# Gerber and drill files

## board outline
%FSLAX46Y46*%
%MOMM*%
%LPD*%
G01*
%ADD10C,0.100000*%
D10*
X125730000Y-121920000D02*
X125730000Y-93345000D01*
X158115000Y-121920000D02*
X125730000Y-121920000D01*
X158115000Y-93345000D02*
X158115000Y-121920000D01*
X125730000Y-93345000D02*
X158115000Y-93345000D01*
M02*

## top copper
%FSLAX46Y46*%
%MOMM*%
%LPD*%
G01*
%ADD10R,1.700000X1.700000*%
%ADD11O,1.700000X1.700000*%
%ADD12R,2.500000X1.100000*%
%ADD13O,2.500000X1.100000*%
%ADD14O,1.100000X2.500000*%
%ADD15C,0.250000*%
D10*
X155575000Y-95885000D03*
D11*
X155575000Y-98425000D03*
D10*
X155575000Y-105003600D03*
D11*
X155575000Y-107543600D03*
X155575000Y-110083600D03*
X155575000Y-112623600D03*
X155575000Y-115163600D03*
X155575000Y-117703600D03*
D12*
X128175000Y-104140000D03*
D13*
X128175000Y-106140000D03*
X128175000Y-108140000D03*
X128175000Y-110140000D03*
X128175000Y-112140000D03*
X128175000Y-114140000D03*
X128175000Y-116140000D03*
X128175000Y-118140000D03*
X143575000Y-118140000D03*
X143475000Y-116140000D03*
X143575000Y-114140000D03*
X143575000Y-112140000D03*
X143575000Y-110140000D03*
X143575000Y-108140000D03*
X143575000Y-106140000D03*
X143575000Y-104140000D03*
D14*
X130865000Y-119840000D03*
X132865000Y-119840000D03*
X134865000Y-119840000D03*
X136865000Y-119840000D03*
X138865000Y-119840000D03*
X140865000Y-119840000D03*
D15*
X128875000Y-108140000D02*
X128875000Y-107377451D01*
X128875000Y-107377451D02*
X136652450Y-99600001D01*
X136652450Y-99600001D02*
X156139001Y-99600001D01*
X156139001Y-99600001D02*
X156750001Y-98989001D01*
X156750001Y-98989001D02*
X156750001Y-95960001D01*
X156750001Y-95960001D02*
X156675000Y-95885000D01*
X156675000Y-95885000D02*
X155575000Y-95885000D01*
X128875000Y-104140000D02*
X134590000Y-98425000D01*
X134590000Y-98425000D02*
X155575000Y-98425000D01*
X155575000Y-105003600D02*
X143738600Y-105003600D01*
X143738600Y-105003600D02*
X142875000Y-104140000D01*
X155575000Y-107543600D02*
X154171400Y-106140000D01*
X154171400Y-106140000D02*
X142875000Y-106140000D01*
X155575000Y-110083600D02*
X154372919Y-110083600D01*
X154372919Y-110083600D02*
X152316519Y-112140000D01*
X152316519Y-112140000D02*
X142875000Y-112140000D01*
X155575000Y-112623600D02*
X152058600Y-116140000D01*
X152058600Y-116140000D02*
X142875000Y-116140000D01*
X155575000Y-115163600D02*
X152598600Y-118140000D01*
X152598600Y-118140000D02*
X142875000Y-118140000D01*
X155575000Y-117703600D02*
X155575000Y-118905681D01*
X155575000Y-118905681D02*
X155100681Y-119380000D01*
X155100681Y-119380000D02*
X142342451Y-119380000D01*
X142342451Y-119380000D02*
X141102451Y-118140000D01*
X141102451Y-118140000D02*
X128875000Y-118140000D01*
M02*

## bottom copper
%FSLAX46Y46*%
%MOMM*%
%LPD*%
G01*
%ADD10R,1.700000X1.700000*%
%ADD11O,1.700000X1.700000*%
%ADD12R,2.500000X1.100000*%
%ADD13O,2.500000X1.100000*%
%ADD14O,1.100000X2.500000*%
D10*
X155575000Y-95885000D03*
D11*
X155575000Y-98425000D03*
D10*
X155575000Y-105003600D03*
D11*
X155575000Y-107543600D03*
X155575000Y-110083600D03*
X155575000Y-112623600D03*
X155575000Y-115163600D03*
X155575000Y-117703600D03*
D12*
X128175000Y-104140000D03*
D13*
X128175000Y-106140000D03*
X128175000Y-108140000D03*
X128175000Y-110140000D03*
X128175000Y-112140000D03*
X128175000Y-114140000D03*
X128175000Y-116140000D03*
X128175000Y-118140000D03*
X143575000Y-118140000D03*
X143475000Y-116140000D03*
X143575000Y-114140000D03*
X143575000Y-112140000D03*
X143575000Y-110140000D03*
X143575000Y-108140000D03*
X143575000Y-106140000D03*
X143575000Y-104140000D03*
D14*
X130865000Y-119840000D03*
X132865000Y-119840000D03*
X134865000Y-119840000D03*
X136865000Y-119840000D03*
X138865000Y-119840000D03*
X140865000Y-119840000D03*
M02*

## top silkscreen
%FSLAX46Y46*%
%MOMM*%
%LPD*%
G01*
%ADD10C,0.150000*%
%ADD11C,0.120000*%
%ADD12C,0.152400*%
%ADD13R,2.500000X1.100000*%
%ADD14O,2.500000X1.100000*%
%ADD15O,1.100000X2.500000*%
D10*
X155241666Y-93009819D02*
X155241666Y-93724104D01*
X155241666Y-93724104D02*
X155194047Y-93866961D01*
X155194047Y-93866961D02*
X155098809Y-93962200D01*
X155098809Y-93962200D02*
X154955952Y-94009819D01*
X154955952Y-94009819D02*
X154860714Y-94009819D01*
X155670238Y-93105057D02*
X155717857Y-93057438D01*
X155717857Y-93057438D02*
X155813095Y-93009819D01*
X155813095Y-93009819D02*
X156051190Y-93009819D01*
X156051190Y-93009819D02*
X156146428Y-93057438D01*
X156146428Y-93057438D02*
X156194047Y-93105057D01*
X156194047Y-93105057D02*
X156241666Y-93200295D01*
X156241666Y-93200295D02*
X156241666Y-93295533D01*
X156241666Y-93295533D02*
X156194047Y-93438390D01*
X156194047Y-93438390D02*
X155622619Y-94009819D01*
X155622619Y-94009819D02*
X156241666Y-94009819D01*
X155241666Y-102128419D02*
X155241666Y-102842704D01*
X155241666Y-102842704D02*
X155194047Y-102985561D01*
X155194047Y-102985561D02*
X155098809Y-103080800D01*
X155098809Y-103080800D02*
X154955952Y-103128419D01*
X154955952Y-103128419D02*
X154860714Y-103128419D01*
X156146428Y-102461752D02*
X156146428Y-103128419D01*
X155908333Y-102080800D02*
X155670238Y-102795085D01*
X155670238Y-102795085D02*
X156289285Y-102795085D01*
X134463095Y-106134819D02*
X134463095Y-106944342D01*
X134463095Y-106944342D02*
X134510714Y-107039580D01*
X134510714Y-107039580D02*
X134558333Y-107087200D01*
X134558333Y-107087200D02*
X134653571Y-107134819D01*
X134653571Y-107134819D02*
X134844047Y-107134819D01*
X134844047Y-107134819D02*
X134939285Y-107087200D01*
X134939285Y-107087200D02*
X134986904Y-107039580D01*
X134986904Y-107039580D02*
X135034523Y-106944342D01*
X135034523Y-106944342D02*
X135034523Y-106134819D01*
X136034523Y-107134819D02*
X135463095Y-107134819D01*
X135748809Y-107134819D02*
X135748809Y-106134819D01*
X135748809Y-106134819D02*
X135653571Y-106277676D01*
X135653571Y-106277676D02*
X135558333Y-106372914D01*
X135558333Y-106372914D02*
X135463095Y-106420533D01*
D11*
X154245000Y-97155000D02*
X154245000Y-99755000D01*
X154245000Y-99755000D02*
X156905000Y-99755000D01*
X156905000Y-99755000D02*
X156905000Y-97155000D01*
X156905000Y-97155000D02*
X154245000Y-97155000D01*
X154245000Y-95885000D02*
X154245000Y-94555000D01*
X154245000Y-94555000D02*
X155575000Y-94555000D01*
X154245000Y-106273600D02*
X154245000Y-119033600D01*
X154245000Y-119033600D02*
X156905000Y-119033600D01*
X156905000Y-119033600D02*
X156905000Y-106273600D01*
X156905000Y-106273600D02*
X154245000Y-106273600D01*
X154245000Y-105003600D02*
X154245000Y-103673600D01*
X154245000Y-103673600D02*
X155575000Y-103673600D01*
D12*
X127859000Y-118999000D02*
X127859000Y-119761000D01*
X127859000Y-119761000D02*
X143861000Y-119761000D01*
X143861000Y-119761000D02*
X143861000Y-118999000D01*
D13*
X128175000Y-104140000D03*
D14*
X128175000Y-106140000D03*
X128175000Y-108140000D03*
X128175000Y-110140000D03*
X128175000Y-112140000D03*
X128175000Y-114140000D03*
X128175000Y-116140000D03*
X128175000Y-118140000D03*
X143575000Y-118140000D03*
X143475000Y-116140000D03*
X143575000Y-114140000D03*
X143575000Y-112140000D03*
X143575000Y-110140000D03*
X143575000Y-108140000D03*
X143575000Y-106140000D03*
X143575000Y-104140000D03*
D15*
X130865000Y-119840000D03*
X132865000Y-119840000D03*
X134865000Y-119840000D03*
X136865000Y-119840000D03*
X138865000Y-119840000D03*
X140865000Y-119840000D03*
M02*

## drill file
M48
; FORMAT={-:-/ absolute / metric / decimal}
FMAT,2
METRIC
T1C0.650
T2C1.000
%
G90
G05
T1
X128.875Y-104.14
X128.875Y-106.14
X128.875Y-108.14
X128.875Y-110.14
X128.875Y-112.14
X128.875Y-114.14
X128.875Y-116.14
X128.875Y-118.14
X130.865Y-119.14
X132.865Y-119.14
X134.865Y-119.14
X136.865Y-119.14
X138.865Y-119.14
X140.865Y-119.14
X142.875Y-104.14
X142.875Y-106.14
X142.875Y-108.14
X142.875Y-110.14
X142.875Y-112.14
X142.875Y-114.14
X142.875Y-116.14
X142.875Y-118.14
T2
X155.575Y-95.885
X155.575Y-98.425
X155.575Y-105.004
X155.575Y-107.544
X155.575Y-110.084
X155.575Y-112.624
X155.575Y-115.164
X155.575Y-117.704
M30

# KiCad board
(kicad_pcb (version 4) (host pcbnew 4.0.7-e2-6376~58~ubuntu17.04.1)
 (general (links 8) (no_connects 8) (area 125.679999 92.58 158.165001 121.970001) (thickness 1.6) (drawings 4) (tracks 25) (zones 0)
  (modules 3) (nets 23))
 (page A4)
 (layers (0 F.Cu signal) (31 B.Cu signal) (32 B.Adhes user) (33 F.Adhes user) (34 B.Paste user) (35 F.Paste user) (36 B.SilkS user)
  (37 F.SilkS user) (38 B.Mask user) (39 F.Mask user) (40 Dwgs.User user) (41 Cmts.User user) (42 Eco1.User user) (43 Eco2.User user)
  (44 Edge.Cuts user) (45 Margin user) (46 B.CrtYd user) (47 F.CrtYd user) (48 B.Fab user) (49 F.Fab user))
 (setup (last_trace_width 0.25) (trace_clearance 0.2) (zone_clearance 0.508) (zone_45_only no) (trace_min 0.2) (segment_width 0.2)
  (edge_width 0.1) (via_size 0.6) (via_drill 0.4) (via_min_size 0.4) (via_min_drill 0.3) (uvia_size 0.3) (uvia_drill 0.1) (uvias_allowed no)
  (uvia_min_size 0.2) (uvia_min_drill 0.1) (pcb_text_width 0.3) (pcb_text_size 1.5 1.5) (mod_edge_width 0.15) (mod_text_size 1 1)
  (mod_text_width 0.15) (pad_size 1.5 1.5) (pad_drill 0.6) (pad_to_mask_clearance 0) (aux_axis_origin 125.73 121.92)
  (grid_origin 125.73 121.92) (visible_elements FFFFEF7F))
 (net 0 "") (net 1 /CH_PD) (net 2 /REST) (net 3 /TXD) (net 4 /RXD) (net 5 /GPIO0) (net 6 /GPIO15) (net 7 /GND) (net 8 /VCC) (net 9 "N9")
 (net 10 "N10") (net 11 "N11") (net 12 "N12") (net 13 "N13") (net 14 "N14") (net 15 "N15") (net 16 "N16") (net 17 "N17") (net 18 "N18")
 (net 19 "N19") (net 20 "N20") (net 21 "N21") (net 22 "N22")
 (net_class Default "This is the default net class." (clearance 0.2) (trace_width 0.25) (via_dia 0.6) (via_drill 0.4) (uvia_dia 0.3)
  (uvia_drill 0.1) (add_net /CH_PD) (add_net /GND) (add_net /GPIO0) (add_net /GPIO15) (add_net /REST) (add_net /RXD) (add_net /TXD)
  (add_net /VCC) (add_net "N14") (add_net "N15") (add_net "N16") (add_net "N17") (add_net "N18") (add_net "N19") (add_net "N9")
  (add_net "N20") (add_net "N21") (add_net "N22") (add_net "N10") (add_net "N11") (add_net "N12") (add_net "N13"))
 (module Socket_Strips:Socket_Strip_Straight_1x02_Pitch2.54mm (layer F.Cu) (at 155.575 95.885)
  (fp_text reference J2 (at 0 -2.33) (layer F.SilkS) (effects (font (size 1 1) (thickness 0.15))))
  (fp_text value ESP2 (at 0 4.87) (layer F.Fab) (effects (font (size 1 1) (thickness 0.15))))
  (fp_line (start -1.33 1.27) (end -1.33 3.87) (layer F.SilkS) (width 0.12))
  (fp_line (start -1.33 3.87) (end 1.33 3.87) (layer F.SilkS) (width 0.12))
  (fp_line (start 1.33 3.87) (end 1.33 1.27) (layer F.SilkS) (width 0.12))
  (fp_line (start 1.33 1.27) (end -1.33 1.27) (layer F.SilkS) (width 0.12))
  (fp_line (start -1.33 0) (end -1.33 -1.33) (layer F.SilkS) (width 0.12))
  (fp_line (start -1.33 -1.33) (end 0 -1.33) (layer F.SilkS) (width 0.12))
  (pad 1 thru_hole rect (at 0 0) (size 1.7 1.7) (drill 1) (layers *.Cu *.Mask) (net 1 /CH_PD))
  (pad 2 thru_hole oval (at 0 2.54) (size 1.7 1.7) (drill 1) (layers *.Cu *.Mask) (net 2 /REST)))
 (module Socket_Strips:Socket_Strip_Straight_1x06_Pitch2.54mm (layer F.Cu) (at 155.575 105.0036)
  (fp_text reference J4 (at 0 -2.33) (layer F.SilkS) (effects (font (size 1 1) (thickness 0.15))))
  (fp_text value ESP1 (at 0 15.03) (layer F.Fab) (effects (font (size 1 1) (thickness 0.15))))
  (fp_line (start -1.33 1.27) (end -1.33 14.03) (layer F.SilkS) (width 0.12))
  (fp_line (start -1.33 14.03) (end 1.33 14.03) (layer F.SilkS) (width 0.12))
  (fp_line (start 1.33 14.03) (end 1.33 1.27) (layer F.SilkS) (width 0.12))
  (fp_line (start 1.33 1.27) (end -1.33 1.27) (layer F.SilkS) (width 0.12))
  (fp_line (start -1.33 0) (end -1.33 -1.33) (layer F.SilkS) (width 0.12))
  (fp_line (start -1.33 -1.33) (end 0 -1.33) (layer F.SilkS) (width 0.12))
  (pad 1 thru_hole rect (at 0 0) (size 1.7 1.7) (drill 1) (layers *.Cu *.Mask) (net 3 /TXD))
  (pad 2 thru_hole oval (at 0 2.54) (size 1.7 1.7) (drill 1) (layers *.Cu *.Mask) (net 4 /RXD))
  (pad 3 thru_hole oval (at 0 5.08) (size 1.7 1.7) (drill 1) (layers *.Cu *.Mask) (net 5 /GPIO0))
  (pad 4 thru_hole oval (at 0 7.62) (size 1.7 1.7) (drill 1) (layers *.Cu *.Mask) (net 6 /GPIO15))
  (pad 5 thru_hole oval (at 0 10.16) (size 1.7 1.7) (drill 1) (layers *.Cu *.Mask) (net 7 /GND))
  (pad 6 thru_hole oval (at 0 12.7) (size 1.7 1.7) (drill 1) (layers *.Cu *.Mask) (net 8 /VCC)))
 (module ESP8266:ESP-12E (layer F.Cu) (at 128.875 104.14)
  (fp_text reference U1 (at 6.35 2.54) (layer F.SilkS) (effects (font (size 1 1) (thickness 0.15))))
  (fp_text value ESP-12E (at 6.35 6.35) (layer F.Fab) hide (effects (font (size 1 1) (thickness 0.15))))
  (fp_line (start -1.016 14.859) (end -1.016 15.621) (layer F.SilkS) (width 0.1524))
  (fp_line (start -1.016 15.621) (end 14.986 15.621) (layer F.SilkS) (width 0.1524))
  (fp_line (start 14.986 15.621) (end 14.986 14.859) (layer F.SilkS) (width 0.1524))
  (pad 1 thru_hole rect (at 0 0) (size 2.5 1.1) (drill 0.65 (offset -0.7 0)) (layers *.Cu *.Mask F.SilkS) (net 2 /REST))
  (pad 2 thru_hole oval (at 0 2) (size 2.5 1.1) (drill 0.65 (offset -0.7 0)) (layers *.Cu *.Mask F.SilkS) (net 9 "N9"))
  (pad 3 thru_hole oval (at 0 4) (size 2.5 1.1) (drill 0.65 (offset -0.7 0)) (layers *.Cu *.Mask F.SilkS) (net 1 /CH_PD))
  (pad 4 thru_hole oval (at 0 6) (size 2.5 1.1) (drill 0.65 (offset -0.7 0)) (layers *.Cu *.Mask F.SilkS) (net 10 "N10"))
  (pad 5 thru_hole oval (at 0 8) (size 2.5 1.1) (drill 0.65 (offset -0.7 0)) (layers *.Cu *.Mask F.SilkS) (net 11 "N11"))
  (pad 6 thru_hole oval (at 0 10) (size 2.5 1.1) (drill 0.65 (offset -0.7 0)) (layers *.Cu *.Mask F.SilkS) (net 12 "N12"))
  (pad 7 thru_hole oval (at 0 12) (size 2.5 1.1) (drill 0.65 (offset -0.7 0)) (layers *.Cu *.Mask F.SilkS) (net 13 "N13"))
  (pad 8 thru_hole oval (at 0 14) (size 2.5 1.1) (drill 0.65 (offset -0.7 0)) (layers *.Cu *.Mask F.SilkS) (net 8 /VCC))
  (pad 9 thru_hole oval (at 14 14) (size 2.5 1.1) (drill 0.65 (offset 0.7 0)) (layers *.Cu *.Mask F.SilkS) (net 7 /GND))
  (pad 10 thru_hole oval (at 14 12) (size 2.5 1.1) (drill 0.65 (offset 0.6 0)) (layers *.Cu *.Mask F.SilkS) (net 6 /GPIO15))
  (pad 11 thru_hole oval (at 14 10) (size 2.5 1.1) (drill 0.65 (offset 0.7 0)) (layers *.Cu *.Mask F.SilkS) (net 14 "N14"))
  (pad 12 thru_hole oval (at 14 8) (size 2.5 1.1) (drill 0.65 (offset 0.7 0)) (layers *.Cu *.Mask F.SilkS) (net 5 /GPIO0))
  (pad 13 thru_hole oval (at 14 6) (size 2.5 1.1) (drill 0.65 (offset 0.7 0)) (layers *.Cu *.Mask F.SilkS) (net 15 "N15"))
  (pad 14 thru_hole oval (at 14 4) (size 2.5 1.1) (drill 0.65 (offset 0.7 0)) (layers *.Cu *.Mask F.SilkS) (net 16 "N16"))
  (pad 15 thru_hole oval (at 14 2) (size 2.5 1.1) (drill 0.65 (offset 0.7 0)) (layers *.Cu *.Mask F.SilkS) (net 4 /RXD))
  (pad 16 thru_hole oval (at 14 0) (size 2.5 1.1) (drill 0.65 (offset 0.7 0)) (layers *.Cu *.Mask F.SilkS) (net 3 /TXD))
  (pad 17 thru_hole oval (at 1.99 15 90) (size 2.5 1.1) (drill 0.65 (offset -0.7 0)) (layers *.Cu *.Mask F.SilkS) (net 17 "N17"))
  (pad 18 thru_hole oval (at 3.99 15 90) (size 2.5 1.1) (drill 0.65 (offset -0.7 0)) (layers *.Cu *.Mask F.SilkS) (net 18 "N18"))
  (pad 19 thru_hole oval (at 5.99 15 90) (size 2.5 1.1) (drill 0.65 (offset -0.7 0)) (layers *.Cu *.Mask F.SilkS) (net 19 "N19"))
  (pad 20 thru_hole oval (at 7.99 15 90) (size 2.5 1.1) (drill 0.65 (offset -0.7 0)) (layers *.Cu *.Mask F.SilkS) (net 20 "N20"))
  (pad 21 thru_hole oval (at 9.99 15 90) (size 2.5 1.1) (drill 0.65 (offset -0.7 0)) (layers *.Cu *.Mask F.SilkS) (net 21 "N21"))
  (pad 22 thru_hole oval (at 11.99 15 90) (size 2.5 1.1) (drill 0.65 (offset -0.7 0)) (layers *.Cu *.Mask F.SilkS) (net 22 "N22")))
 (gr_line (start 125.73 121.92) (end 125.73 93.345) (layer Edge.Cuts) (width 0.1))
 (gr_line (start 158.115 121.92) (end 125.73 121.92) (layer Edge.Cuts) (width 0.1))
 (gr_line (start 158.115 93.345) (end 158.115 121.92) (layer Edge.Cuts) (width 0.1))
 (gr_line (start 125.73 93.345) (end 158.115 93.345) (layer Edge.Cuts) (width 0.1))
 (segment (start 128.875 108.14) (end 128.875 107.377451) (width 0.25) (layer F.Cu) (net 1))
 (segment (start 128.875 107.377451) (end 136.65245 99.600001) (width 0.25) (layer F.Cu) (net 1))
 (segment (start 136.65245 99.600001) (end 156.139001 99.600001) (width 0.25) (layer F.Cu) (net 1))
 (segment (start 156.139001 99.600001) (end 156.750001 98.989001) (width 0.25) (layer F.Cu) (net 1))
 (segment (start 156.750001 98.989001) (end 156.750001 95.960001) (width 0.25) (layer F.Cu) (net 1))
 (segment (start 156.750001 95.960001) (end 156.675 95.885) (width 0.25) (layer F.Cu) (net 1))
 (segment (start 156.675 95.885) (end 155.575 95.885) (width 0.25) (layer F.Cu) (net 1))
 (segment (start 128.875 104.14) (end 134.59 98.425) (width 0.25) (layer F.Cu) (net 2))
 (segment (start 134.59 98.425) (end 155.575 98.425) (width 0.25) (layer F.Cu) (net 2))
 (segment (start 155.575 105.0036) (end 143.7386 105.0036) (width 0.25) (layer F.Cu) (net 3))
 (segment (start 143.7386 105.0036) (end 142.875 104.14) (width 0.25) (layer F.Cu) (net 3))
 (segment (start 155.575 107.5436) (end 154.1714 106.14) (width 0.25) (layer F.Cu) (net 4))
 (segment (start 154.1714 106.14) (end 142.875 106.14) (width 0.25) (layer F.Cu) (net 4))
 (segment (start 155.575 110.0836) (end 154.372919 110.0836) (width 0.25) (layer F.Cu) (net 5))
 (segment (start 154.372919 110.0836) (end 152.316519 112.14) (width 0.25) (layer F.Cu) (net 5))
 (segment (start 152.316519 112.14) (end 142.875 112.14) (width 0.25) (layer F.Cu) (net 5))
 (segment (start 155.575 112.6236) (end 152.0586 116.14) (width 0.25) (layer F.Cu) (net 6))
 (segment (start 152.0586 116.14) (end 142.875 116.14) (width 0.25) (layer F.Cu) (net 6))
 (segment (start 155.575 115.1636) (end 152.5986 118.14) (width 0.25) (layer F.Cu) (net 7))
 (segment (start 152.5986 118.14) (end 142.875 118.14) (width 0.25) (layer F.Cu) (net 7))
 (segment (start 155.575 117.7036) (end 155.575 118.905681) (width 0.25) (layer F.Cu) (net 8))
 (segment (start 155.575 118.905681) (end 155.100681 119.38) (width 0.25) (layer F.Cu) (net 8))
 (segment (start 155.100681 119.38) (end 142.342451 119.38) (width 0.25) (layer F.Cu) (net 8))
 (segment (start 142.342451 119.38) (end 141.102451 118.14) (width 0.25) (layer F.Cu) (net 8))
 (segment (start 141.102451 118.14) (end 128.875 118.14) (width 0.25) (layer F.Cu) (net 8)))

